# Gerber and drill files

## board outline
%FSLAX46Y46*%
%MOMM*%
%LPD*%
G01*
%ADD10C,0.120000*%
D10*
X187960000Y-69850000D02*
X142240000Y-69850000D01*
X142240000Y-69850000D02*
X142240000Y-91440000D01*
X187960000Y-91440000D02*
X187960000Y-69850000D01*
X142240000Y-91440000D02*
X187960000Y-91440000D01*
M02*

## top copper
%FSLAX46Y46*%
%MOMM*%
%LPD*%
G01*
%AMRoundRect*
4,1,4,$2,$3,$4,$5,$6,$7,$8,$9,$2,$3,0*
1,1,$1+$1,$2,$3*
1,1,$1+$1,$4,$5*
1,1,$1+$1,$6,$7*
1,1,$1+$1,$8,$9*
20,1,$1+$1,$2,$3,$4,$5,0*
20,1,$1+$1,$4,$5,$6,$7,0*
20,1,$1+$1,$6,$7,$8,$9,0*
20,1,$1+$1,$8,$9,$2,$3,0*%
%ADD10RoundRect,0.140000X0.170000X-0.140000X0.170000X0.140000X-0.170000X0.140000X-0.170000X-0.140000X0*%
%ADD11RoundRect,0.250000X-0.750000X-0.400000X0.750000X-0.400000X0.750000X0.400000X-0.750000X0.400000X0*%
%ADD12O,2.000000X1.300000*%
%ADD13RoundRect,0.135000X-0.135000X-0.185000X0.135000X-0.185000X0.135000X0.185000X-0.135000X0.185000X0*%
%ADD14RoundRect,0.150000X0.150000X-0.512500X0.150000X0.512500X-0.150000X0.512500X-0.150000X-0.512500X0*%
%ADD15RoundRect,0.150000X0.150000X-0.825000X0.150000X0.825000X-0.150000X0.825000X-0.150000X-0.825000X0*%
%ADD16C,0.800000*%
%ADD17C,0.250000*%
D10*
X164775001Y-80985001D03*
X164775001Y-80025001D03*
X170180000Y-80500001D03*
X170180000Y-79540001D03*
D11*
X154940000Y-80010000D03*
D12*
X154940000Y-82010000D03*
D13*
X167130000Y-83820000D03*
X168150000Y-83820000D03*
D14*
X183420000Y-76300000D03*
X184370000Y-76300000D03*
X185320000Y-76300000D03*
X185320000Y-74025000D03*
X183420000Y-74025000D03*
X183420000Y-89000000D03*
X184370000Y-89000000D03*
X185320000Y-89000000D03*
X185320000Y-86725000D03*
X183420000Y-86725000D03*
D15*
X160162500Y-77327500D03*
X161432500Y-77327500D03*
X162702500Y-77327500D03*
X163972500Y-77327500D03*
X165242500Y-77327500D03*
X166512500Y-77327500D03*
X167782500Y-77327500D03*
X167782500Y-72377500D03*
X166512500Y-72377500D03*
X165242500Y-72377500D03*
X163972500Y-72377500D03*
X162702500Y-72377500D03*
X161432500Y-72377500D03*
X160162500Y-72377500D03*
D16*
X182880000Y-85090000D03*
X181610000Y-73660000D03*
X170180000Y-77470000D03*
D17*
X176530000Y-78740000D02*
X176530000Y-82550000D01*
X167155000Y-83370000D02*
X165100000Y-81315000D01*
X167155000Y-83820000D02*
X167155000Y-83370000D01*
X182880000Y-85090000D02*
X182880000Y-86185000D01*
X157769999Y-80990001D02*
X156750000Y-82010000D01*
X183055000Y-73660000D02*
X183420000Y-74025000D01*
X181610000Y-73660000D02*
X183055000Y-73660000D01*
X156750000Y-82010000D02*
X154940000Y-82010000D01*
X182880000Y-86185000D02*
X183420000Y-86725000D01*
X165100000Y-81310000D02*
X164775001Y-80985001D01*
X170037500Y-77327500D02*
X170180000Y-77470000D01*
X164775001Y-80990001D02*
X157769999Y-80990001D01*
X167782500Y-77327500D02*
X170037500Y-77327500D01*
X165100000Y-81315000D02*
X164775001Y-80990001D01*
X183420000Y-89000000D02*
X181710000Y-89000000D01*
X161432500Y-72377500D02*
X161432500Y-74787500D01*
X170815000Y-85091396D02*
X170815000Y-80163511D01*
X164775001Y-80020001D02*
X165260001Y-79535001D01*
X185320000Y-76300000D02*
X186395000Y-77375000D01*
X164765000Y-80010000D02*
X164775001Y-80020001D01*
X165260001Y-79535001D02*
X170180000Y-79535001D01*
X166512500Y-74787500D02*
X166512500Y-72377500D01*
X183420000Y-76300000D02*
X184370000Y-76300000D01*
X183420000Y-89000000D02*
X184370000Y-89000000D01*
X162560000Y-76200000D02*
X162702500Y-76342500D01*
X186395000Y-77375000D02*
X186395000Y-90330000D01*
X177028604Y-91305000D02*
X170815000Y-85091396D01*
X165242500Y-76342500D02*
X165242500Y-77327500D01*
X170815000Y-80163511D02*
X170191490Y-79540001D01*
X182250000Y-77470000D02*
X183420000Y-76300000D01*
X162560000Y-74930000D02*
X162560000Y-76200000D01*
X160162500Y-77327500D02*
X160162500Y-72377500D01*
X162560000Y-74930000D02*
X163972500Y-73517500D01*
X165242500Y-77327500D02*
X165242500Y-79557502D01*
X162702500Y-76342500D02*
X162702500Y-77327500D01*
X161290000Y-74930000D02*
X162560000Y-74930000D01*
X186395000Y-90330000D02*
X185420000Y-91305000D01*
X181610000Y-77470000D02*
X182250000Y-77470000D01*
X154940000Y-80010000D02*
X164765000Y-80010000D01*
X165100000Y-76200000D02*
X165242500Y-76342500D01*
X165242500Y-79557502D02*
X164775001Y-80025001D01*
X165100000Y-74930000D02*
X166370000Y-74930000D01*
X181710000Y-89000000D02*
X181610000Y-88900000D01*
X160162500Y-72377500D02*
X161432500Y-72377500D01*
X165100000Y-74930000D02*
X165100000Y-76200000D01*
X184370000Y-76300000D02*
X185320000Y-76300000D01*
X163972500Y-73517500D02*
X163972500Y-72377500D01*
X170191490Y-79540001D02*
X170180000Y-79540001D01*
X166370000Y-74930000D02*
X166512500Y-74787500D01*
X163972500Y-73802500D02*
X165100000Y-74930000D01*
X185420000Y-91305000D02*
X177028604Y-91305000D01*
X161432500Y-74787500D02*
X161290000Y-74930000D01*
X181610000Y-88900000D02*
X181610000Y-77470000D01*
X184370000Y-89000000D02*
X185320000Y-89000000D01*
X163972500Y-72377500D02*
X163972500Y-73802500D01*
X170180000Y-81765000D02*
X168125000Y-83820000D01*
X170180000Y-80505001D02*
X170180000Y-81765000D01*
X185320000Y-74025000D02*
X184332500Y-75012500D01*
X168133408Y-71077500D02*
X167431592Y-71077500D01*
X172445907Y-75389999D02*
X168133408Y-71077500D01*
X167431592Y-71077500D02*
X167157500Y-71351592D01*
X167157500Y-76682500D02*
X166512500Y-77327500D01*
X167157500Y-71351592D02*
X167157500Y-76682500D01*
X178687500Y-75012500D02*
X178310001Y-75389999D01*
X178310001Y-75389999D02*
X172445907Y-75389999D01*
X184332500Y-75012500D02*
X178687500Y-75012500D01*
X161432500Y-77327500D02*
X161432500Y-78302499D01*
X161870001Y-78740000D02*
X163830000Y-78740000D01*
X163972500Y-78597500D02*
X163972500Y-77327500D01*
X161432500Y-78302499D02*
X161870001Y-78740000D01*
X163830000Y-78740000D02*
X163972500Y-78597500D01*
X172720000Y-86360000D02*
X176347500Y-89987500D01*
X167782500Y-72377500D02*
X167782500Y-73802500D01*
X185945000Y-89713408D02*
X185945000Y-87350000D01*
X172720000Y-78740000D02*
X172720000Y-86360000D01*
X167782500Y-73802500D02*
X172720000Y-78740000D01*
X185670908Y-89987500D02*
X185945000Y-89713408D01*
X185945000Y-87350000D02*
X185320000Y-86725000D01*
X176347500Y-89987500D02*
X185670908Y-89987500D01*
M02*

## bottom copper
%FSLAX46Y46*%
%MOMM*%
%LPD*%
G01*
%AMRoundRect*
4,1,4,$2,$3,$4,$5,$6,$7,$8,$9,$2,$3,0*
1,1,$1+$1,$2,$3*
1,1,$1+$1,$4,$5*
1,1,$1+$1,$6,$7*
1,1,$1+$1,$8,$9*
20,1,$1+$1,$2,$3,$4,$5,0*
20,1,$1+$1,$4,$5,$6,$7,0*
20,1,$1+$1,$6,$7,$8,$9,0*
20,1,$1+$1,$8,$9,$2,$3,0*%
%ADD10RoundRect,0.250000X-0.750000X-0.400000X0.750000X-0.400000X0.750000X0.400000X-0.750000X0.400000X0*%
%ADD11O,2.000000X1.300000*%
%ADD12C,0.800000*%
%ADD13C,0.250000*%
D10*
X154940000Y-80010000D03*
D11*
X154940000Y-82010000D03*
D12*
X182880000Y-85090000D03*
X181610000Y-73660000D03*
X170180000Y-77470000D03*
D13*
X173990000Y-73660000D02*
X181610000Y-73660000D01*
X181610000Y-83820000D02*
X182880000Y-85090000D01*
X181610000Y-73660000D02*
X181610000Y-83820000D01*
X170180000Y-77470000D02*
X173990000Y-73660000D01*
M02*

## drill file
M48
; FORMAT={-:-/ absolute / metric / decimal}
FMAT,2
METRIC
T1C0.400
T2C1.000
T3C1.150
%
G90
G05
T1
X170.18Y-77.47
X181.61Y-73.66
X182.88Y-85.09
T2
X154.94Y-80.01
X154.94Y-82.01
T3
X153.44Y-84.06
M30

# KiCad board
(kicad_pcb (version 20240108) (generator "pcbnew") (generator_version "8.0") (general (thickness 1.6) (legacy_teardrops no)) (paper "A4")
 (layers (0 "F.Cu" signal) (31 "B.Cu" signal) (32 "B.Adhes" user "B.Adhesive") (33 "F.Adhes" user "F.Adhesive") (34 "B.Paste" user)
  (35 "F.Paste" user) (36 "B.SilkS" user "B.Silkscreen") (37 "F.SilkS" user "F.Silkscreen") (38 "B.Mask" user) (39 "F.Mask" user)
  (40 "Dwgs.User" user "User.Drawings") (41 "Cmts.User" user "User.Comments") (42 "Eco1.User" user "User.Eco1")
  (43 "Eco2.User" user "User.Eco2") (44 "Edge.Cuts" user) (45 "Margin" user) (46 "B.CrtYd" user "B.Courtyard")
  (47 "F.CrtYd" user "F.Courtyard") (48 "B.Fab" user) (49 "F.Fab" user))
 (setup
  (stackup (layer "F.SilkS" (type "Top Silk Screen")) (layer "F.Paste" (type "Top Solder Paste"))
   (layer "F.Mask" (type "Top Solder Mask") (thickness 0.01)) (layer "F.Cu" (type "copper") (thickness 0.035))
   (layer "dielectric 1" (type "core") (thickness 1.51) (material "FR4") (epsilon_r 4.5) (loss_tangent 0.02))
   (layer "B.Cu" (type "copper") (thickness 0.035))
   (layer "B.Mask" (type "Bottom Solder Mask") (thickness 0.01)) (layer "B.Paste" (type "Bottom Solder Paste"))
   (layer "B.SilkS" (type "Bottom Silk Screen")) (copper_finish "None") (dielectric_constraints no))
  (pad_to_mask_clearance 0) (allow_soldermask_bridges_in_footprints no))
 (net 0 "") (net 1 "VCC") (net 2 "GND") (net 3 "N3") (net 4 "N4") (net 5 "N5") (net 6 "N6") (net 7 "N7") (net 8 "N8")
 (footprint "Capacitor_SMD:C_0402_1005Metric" (layer "F.Cu") (at 164.775001 80.505001 90)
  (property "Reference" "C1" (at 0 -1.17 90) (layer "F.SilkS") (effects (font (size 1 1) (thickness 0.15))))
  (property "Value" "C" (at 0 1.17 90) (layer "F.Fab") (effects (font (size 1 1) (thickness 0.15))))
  (pad "1" smd roundrect (at -0.48 0 90) (size 0.56 0.62) (layers "F.Cu" "F.Paste" "F.Mask") (roundrect_rratio 0.25) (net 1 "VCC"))
  (pad "2" smd roundrect (at 0.48 0 90) (size 0.56 0.62) (layers "F.Cu" "F.Paste" "F.Mask") (roundrect_rratio 0.25) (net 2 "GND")))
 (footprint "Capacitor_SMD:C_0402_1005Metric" (layer "F.Cu") (at 170.18 80.020001 90)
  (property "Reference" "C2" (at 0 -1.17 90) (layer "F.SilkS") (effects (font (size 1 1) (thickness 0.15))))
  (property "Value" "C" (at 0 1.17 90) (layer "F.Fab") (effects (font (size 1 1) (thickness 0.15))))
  (pad "1" smd roundrect (at -0.48 0 90) (size 0.56 0.62) (layers "F.Cu" "F.Paste" "F.Mask") (roundrect_rratio 0.25) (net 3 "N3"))
  (pad "2" smd roundrect (at 0.48 0 90) (size 0.56 0.62) (layers "F.Cu" "F.Paste" "F.Mask") (roundrect_rratio 0.25) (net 2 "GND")))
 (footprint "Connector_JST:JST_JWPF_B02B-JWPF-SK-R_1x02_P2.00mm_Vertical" (layer "F.Cu") (at 154.94 80.01)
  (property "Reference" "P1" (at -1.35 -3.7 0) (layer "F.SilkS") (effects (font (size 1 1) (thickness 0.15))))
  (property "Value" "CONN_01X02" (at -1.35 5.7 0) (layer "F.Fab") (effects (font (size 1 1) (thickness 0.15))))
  (pad "" np_thru_hole circle (at -1.5 4.05) (size 1.15 1.15) (drill 1.15) (layers "*.Cu" "*.Mask"))
  (pad "1" thru_hole roundrect (at 0 0) (size 2 1.3) (drill 1) (layers "*.Cu" "*.Mask") (remove_unused_layers no)
   (roundrect_rratio 0.192308) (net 2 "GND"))
  (pad "2" thru_hole oval (at 0 2) (size 2 1.3) (drill 1) (layers "*.Cu" "*.Mask") (remove_unused_layers no) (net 1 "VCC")))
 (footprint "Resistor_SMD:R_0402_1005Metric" (layer "F.Cu") (at 167.64 83.82)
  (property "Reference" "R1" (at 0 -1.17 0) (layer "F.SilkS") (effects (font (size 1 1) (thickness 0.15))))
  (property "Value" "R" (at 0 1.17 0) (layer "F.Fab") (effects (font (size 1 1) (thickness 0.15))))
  (pad "1" smd roundrect (at -0.51 0) (size 0.54 0.64) (layers "F.Cu" "F.Paste" "F.Mask") (roundrect_rratio 0.25) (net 1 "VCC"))
  (pad "2" smd roundrect (at 0.51 0) (size 0.54 0.64) (layers "F.Cu" "F.Paste" "F.Mask") (roundrect_rratio 0.25) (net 3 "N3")))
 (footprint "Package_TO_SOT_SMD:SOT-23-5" (layer "F.Cu") (at 184.37 75.1625 90)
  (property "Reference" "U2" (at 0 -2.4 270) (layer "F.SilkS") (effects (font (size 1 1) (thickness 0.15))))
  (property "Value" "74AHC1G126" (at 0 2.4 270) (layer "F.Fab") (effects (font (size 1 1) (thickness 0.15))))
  (pad "1" smd roundrect (at -1.1375 -0.95 90) (size 1.325 0.6) (layers "F.Cu" "F.Paste" "F.Mask") (roundrect_rratio 0.25) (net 2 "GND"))
  (pad "2" smd roundrect (at -1.1375 0 90) (size 1.325 0.6) (layers "F.Cu" "F.Paste" "F.Mask") (roundrect_rratio 0.25) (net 2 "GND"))
  (pad "3" smd roundrect (at -1.1375 0.95 90) (size 1.325 0.6) (layers "F.Cu" "F.Paste" "F.Mask") (roundrect_rratio 0.25) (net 2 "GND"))
  (pad "4" smd roundrect (at 1.1375 0.95 90) (size 1.325 0.6) (layers "F.Cu" "F.Paste" "F.Mask") (roundrect_rratio 0.25) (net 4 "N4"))
  (pad "5" smd roundrect (at 1.1375 -0.95 90) (size 1.325 0.6) (layers "F.Cu" "F.Paste" "F.Mask") (roundrect_rratio 0.25) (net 1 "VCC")))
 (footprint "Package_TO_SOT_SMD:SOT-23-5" (layer "F.Cu") (at 184.37 87.8625 90)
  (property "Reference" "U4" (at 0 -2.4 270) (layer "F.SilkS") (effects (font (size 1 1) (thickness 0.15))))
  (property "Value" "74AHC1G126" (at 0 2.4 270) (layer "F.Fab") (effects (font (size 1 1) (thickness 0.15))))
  (pad "1" smd roundrect (at -1.1375 -0.95 90) (size 1.325 0.6) (layers "F.Cu" "F.Paste" "F.Mask") (roundrect_rratio 0.25) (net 2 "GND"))
  (pad "2" smd roundrect (at -1.1375 0 90) (size 1.325 0.6) (layers "F.Cu" "F.Paste" "F.Mask") (roundrect_rratio 0.25) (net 2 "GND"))
  (pad "3" smd roundrect (at -1.1375 0.95 90) (size 1.325 0.6) (layers "F.Cu" "F.Paste" "F.Mask") (roundrect_rratio 0.25) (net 2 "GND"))
  (pad "4" smd roundrect (at 1.1375 0.95 90) (size 1.325 0.6) (layers "F.Cu" "F.Paste" "F.Mask") (roundrect_rratio 0.25) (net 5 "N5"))
  (pad "5" smd roundrect (at 1.1375 -0.95 90) (size 1.325 0.6) (layers "F.Cu" "F.Paste" "F.Mask") (roundrect_rratio 0.25) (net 1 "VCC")))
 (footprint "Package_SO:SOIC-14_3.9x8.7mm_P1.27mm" (layer "F.Cu") (at 163.9725 74.8525 90)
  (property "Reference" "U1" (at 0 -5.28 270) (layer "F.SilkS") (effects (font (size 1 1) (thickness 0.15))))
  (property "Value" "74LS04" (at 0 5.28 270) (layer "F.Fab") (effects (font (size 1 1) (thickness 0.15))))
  (pad "1" smd roundrect (at -2.475 -3.81 90) (size 1.95 0.6) (layers "F.Cu" "F.Paste" "F.Mask") (roundrect_rratio 0.25) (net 2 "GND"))
  (pad "2" smd roundrect (at -2.475 -2.54 90) (size 1.95 0.6) (layers "F.Cu" "F.Paste" "F.Mask") (roundrect_rratio 0.25) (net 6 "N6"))
  (pad "3" smd roundrect (at -2.475 -1.27 90) (size 1.95 0.6) (layers "F.Cu" "F.Paste" "F.Mask") (roundrect_rratio 0.25) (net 2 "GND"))
  (pad "4" smd roundrect (at -2.475 0 90) (size 1.95 0.6) (layers "F.Cu" "F.Paste" "F.Mask") (roundrect_rratio 0.25) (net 6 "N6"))
  (pad "5" smd roundrect (at -2.475 1.27 90) (size 1.95 0.6) (layers "F.Cu" "F.Paste" "F.Mask") (roundrect_rratio 0.25) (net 2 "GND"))
  (pad "6" smd roundrect (at -2.475 2.54 90) (size 1.95 0.6) (layers "F.Cu" "F.Paste" "F.Mask") (roundrect_rratio 0.25) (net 4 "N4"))
  (pad "7" smd roundrect (at -2.475 3.81 90) (size 1.95 0.6) (layers "F.Cu" "F.Paste" "F.Mask") (roundrect_rratio 0.25) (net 1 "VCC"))
  (pad "8" smd roundrect (at 2.475 3.81 90) (size 1.95 0.6) (layers "F.Cu" "F.Paste" "F.Mask") (roundrect_rratio 0.25) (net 5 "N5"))
  (pad "9" smd roundrect (at 2.475 2.54 90) (size 1.95 0.6) (layers "F.Cu" "F.Paste" "F.Mask") (roundrect_rratio 0.25) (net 2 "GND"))
  (pad "10" smd roundrect (at 2.475 1.27 90) (size 1.95 0.6) (layers "F.Cu" "F.Paste" "F.Mask") (roundrect_rratio 0.25) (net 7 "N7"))
  (pad "11" smd roundrect (at 2.475 0 90) (size 1.95 0.6) (layers "F.Cu" "F.Paste" "F.Mask") (roundrect_rratio 0.25) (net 2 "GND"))
  (pad "12" smd roundrect (at 2.475 -1.27 90) (size 1.95 0.6) (layers "F.Cu" "F.Paste" "F.Mask") (roundrect_rratio 0.25) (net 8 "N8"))
  (pad "13" smd roundrect (at 2.475 -2.54 90) (size 1.95 0.6) (layers "F.Cu" "F.Paste" "F.Mask") (roundrect_rratio 0.25) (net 2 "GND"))
  (pad "14" smd roundrect (at 2.475 -3.81 90) (size 1.95 0.6) (layers "F.Cu" "F.Paste" "F.Mask") (roundrect_rratio 0.25) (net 2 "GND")))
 (gr_line (start 187.96 69.85) (end 142.24 69.85) (stroke (width 0.12) (type solid)) (layer "Edge.Cuts"))
 (gr_line (start 142.24 69.85) (end 142.24 91.44) (stroke (width 0.12) (type solid)) (layer "Edge.Cuts"))
 (gr_line (start 187.96 91.44) (end 187.96 69.85) (stroke (width 0.12) (type solid)) (layer "Edge.Cuts"))
 (gr_line (start 142.24 91.44) (end 187.96 91.44) (stroke (width 0.12) (type solid)) (layer "Edge.Cuts"))
 (segment (start 176.53 78.74) (end 176.53 82.55) (width 0.25) (layer "F.Cu") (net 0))
 (segment (start 167.155 83.37) (end 165.1 81.315) (width 0.25) (layer "F.Cu") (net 1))
 (segment (start 167.155 83.82) (end 167.155 83.37) (width 0.25) (layer "F.Cu") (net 1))
 (segment (start 182.88 85.09) (end 182.88 86.185) (width 0.25) (layer "F.Cu") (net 1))
 (segment (start 157.769999 80.990001) (end 156.75 82.01) (width 0.25) (layer "F.Cu") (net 1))
 (segment (start 183.055 73.66) (end 183.42 74.025) (width 0.25) (layer "F.Cu") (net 1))
 (segment (start 181.61 73.66) (end 183.055 73.66) (width 0.25) (layer "F.Cu") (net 1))
 (segment (start 156.75 82.01) (end 154.94 82.01) (width 0.25) (layer "F.Cu") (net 1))
 (segment (start 182.88 86.185) (end 183.42 86.725) (width 0.25) (layer "F.Cu") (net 1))
 (segment (start 165.1 81.31) (end 164.775001 80.985001) (width 0.25) (layer "F.Cu") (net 1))
 (segment (start 170.0375 77.3275) (end 170.18 77.47) (width 0.25) (layer "F.Cu") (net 1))
 (segment (start 164.775001 80.990001) (end 157.769999 80.990001) (width 0.25) (layer "F.Cu") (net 1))
 (segment (start 167.7825 77.3275) (end 170.0375 77.3275) (width 0.25) (layer "F.Cu") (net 1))
 (segment (start 165.1 81.315) (end 164.775001 80.990001) (width 0.25) (layer "F.Cu") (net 1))
 (via (at 182.88 85.09) (size 0.8) (drill 0.4) (layers "F.Cu" "B.Cu") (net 1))
 (via (at 181.61 73.66) (size 0.8) (drill 0.4) (layers "F.Cu" "B.Cu") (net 1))
 (via (at 170.18 77.47) (size 0.8) (drill 0.4) (layers "F.Cu" "B.Cu") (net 1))
 (segment (start 173.99 73.66) (end 181.61 73.66) (width 0.25) (layer "B.Cu") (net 1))
 (segment (start 181.61 83.82) (end 182.88 85.09) (width 0.25) (layer "B.Cu") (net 1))
 (segment (start 181.61 73.66) (end 181.61 83.82) (width 0.25) (layer "B.Cu") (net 1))
 (segment (start 170.18 77.47) (end 173.99 73.66) (width 0.25) (layer "B.Cu") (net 1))
 (segment (start 183.42 89) (end 181.71 89) (width 0.25) (layer "F.Cu") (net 2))
 (segment (start 161.4325 72.3775) (end 161.4325 74.7875) (width 0.25) (layer "F.Cu") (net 2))
 (segment (start 170.815 85.091396) (end 170.815 80.163511) (width 0.25) (layer "F.Cu") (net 2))
 (segment (start 164.775001 80.020001) (end 165.260001 79.535001) (width 0.25) (layer "F.Cu") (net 2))
 (segment (start 185.32 76.3) (end 186.395 77.375) (width 0.25) (layer "F.Cu") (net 2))
 (segment (start 164.765 80.01) (end 164.775001 80.020001) (width 0.25) (layer "F.Cu") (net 2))
 (segment (start 165.260001 79.535001) (end 170.18 79.535001) (width 0.25) (layer "F.Cu") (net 2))
 (segment (start 166.5125 74.7875) (end 166.5125 72.3775) (width 0.25) (layer "F.Cu") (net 2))
 (segment (start 183.42 76.3) (end 184.37 76.3) (width 0.25) (layer "F.Cu") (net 2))
 (segment (start 183.42 89) (end 184.37 89) (width 0.25) (layer "F.Cu") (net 2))
 (segment (start 162.56 76.2) (end 162.7025 76.3425) (width 0.25) (layer "F.Cu") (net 2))
 (segment (start 186.395 77.375) (end 186.395 90.33) (width 0.25) (layer "F.Cu") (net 2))
 (segment (start 177.028604 91.305) (end 170.815 85.091396) (width 0.25) (layer "F.Cu") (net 2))
 (segment (start 165.2425 76.3425) (end 165.2425 77.3275) (width 0.25) (layer "F.Cu") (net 2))
 (segment (start 170.815 80.163511) (end 170.19149 79.540001) (width 0.25) (layer "F.Cu") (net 2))
 (segment (start 182.25 77.47) (end 183.42 76.3) (width 0.25) (layer "F.Cu") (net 2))
 (segment (start 162.56 74.93) (end 162.56 76.2) (width 0.25) (layer "F.Cu") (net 2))
 (segment (start 160.1625 77.3275) (end 160.1625 72.3775) (width 0.25) (layer "F.Cu") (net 2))
 (segment (start 162.56 74.93) (end 163.9725 73.5175) (width 0.25) (layer "F.Cu") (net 2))
 (segment (start 165.2425 77.3275) (end 165.2425 79.557502) (width 0.25) (layer "F.Cu") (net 2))
 (segment (start 162.7025 76.3425) (end 162.7025 77.3275) (width 0.25) (layer "F.Cu") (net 2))
 (segment (start 161.29 74.93) (end 162.56 74.93) (width 0.25) (layer "F.Cu") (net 2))
 (segment (start 186.395 90.33) (end 185.42 91.305) (width 0.25) (layer "F.Cu") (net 2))
 (segment (start 181.61 77.47) (end 182.25 77.47) (width 0.25) (layer "F.Cu") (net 2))
 (segment (start 154.94 80.01) (end 164.765 80.01) (width 0.25) (layer "F.Cu") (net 2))
 (segment (start 165.1 76.2) (end 165.2425 76.3425) (width 0.25) (layer "F.Cu") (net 2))
 (segment (start 165.2425 79.557502) (end 164.775001 80.025001) (width 0.25) (layer "F.Cu") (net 2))
 (segment (start 165.1 74.93) (end 166.37 74.93) (width 0.25) (layer "F.Cu") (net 2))
 (segment (start 181.71 89) (end 181.61 88.9) (width 0.25) (layer "F.Cu") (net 2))
 (segment (start 160.1625 72.3775) (end 161.4325 72.3775) (width 0.25) (layer "F.Cu") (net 2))
 (segment (start 165.1 74.93) (end 165.1 76.2) (width 0.25) (layer "F.Cu") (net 2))
 (segment (start 184.37 76.3) (end 185.32 76.3) (width 0.25) (layer "F.Cu") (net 2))
 (segment (start 163.9725 73.5175) (end 163.9725 72.3775) (width 0.25) (layer "F.Cu") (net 2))
 (segment (start 170.19149 79.540001) (end 170.18 79.540001) (width 0.25) (layer "F.Cu") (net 2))
 (segment (start 166.37 74.93) (end 166.5125 74.7875) (width 0.25) (layer "F.Cu") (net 2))
 (segment (start 163.9725 73.8025) (end 165.1 74.93) (width 0.25) (layer "F.Cu") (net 2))
 (segment (start 185.42 91.305) (end 177.028604 91.305) (width 0.25) (layer "F.Cu") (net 2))
 (segment (start 161.4325 74.7875) (end 161.29 74.93) (width 0.25) (layer "F.Cu") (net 2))
 (segment (start 181.61 88.9) (end 181.61 77.47) (width 0.25) (layer "F.Cu") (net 2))
 (segment (start 184.37 89) (end 185.32 89) (width 0.25) (layer "F.Cu") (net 2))
 (segment (start 163.9725 72.3775) (end 163.9725 73.8025) (width 0.25) (layer "F.Cu") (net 2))
 (segment (start 170.18 81.765) (end 168.125 83.82) (width 0.25) (layer "F.Cu") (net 3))
 (segment (start 170.18 80.505001) (end 170.18 81.765) (width 0.25) (layer "F.Cu") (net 3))
 (segment (start 185.32 74.025) (end 184.3325 75.0125) (width 0.25) (layer "F.Cu") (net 4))
 (segment (start 168.133408 71.0775) (end 167.431592 71.0775) (width 0.25) (layer "F.Cu") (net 4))
 (segment (start 172.445907 75.389999) (end 168.133408 71.0775) (width 0.25) (layer "F.Cu") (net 4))
 (segment (start 167.431592 71.0775) (end 167.1575 71.351592) (width 0.25) (layer "F.Cu") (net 4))
 (segment (start 167.1575 76.6825) (end 166.5125 77.3275) (width 0.25) (layer "F.Cu") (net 4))
 (segment (start 167.1575 71.351592) (end 167.1575 76.6825) (width 0.25) (layer "F.Cu") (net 4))
 (segment (start 178.6875 75.0125) (end 178.310001 75.389999) (width 0.25) (layer "F.Cu") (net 4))
 (segment (start 178.310001 75.389999) (end 172.445907 75.389999) (width 0.25) (layer "F.Cu") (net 4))
 (segment (start 184.3325 75.0125) (end 178.6875 75.0125) (width 0.25) (layer "F.Cu") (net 4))
 (segment (start 161.4325 77.3275) (end 161.4325 78.302499) (width 0.25) (layer "F.Cu") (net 6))
 (segment (start 161.870001 78.74) (end 163.83 78.74) (width 0.25) (layer "F.Cu") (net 6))
 (segment (start 163.9725 78.5975) (end 163.9725 77.3275) (width 0.25) (layer "F.Cu") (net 6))
 (segment (start 161.4325 78.302499) (end 161.870001 78.74) (width 0.25) (layer "F.Cu") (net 6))
 (segment (start 163.83 78.74) (end 163.9725 78.5975) (width 0.25) (layer "F.Cu") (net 6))
 (segment (start 172.72 86.36) (end 176.3475 89.9875) (width 0.25) (layer "F.Cu") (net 5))
 (segment (start 167.7825 72.3775) (end 167.7825 73.8025) (width 0.25) (layer "F.Cu") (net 5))
 (segment (start 185.945 89.713408) (end 185.945 87.35) (width 0.25) (layer "F.Cu") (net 5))
 (segment (start 172.72 78.74) (end 172.72 86.36) (width 0.25) (layer "F.Cu") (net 5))
 (segment (start 167.7825 73.8025) (end 172.72 78.74) (width 0.25) (layer "F.Cu") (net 5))
 (segment (start 185.670908 89.9875) (end 185.945 89.713408) (width 0.25) (layer "F.Cu") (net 5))
 (segment (start 185.945 87.35) (end 185.32 86.725) (width 0.25) (layer "F.Cu") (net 5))
 (segment (start 176.3475 89.9875) (end 185.670908 89.9875) (width 0.25) (layer "F.Cu") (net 5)))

